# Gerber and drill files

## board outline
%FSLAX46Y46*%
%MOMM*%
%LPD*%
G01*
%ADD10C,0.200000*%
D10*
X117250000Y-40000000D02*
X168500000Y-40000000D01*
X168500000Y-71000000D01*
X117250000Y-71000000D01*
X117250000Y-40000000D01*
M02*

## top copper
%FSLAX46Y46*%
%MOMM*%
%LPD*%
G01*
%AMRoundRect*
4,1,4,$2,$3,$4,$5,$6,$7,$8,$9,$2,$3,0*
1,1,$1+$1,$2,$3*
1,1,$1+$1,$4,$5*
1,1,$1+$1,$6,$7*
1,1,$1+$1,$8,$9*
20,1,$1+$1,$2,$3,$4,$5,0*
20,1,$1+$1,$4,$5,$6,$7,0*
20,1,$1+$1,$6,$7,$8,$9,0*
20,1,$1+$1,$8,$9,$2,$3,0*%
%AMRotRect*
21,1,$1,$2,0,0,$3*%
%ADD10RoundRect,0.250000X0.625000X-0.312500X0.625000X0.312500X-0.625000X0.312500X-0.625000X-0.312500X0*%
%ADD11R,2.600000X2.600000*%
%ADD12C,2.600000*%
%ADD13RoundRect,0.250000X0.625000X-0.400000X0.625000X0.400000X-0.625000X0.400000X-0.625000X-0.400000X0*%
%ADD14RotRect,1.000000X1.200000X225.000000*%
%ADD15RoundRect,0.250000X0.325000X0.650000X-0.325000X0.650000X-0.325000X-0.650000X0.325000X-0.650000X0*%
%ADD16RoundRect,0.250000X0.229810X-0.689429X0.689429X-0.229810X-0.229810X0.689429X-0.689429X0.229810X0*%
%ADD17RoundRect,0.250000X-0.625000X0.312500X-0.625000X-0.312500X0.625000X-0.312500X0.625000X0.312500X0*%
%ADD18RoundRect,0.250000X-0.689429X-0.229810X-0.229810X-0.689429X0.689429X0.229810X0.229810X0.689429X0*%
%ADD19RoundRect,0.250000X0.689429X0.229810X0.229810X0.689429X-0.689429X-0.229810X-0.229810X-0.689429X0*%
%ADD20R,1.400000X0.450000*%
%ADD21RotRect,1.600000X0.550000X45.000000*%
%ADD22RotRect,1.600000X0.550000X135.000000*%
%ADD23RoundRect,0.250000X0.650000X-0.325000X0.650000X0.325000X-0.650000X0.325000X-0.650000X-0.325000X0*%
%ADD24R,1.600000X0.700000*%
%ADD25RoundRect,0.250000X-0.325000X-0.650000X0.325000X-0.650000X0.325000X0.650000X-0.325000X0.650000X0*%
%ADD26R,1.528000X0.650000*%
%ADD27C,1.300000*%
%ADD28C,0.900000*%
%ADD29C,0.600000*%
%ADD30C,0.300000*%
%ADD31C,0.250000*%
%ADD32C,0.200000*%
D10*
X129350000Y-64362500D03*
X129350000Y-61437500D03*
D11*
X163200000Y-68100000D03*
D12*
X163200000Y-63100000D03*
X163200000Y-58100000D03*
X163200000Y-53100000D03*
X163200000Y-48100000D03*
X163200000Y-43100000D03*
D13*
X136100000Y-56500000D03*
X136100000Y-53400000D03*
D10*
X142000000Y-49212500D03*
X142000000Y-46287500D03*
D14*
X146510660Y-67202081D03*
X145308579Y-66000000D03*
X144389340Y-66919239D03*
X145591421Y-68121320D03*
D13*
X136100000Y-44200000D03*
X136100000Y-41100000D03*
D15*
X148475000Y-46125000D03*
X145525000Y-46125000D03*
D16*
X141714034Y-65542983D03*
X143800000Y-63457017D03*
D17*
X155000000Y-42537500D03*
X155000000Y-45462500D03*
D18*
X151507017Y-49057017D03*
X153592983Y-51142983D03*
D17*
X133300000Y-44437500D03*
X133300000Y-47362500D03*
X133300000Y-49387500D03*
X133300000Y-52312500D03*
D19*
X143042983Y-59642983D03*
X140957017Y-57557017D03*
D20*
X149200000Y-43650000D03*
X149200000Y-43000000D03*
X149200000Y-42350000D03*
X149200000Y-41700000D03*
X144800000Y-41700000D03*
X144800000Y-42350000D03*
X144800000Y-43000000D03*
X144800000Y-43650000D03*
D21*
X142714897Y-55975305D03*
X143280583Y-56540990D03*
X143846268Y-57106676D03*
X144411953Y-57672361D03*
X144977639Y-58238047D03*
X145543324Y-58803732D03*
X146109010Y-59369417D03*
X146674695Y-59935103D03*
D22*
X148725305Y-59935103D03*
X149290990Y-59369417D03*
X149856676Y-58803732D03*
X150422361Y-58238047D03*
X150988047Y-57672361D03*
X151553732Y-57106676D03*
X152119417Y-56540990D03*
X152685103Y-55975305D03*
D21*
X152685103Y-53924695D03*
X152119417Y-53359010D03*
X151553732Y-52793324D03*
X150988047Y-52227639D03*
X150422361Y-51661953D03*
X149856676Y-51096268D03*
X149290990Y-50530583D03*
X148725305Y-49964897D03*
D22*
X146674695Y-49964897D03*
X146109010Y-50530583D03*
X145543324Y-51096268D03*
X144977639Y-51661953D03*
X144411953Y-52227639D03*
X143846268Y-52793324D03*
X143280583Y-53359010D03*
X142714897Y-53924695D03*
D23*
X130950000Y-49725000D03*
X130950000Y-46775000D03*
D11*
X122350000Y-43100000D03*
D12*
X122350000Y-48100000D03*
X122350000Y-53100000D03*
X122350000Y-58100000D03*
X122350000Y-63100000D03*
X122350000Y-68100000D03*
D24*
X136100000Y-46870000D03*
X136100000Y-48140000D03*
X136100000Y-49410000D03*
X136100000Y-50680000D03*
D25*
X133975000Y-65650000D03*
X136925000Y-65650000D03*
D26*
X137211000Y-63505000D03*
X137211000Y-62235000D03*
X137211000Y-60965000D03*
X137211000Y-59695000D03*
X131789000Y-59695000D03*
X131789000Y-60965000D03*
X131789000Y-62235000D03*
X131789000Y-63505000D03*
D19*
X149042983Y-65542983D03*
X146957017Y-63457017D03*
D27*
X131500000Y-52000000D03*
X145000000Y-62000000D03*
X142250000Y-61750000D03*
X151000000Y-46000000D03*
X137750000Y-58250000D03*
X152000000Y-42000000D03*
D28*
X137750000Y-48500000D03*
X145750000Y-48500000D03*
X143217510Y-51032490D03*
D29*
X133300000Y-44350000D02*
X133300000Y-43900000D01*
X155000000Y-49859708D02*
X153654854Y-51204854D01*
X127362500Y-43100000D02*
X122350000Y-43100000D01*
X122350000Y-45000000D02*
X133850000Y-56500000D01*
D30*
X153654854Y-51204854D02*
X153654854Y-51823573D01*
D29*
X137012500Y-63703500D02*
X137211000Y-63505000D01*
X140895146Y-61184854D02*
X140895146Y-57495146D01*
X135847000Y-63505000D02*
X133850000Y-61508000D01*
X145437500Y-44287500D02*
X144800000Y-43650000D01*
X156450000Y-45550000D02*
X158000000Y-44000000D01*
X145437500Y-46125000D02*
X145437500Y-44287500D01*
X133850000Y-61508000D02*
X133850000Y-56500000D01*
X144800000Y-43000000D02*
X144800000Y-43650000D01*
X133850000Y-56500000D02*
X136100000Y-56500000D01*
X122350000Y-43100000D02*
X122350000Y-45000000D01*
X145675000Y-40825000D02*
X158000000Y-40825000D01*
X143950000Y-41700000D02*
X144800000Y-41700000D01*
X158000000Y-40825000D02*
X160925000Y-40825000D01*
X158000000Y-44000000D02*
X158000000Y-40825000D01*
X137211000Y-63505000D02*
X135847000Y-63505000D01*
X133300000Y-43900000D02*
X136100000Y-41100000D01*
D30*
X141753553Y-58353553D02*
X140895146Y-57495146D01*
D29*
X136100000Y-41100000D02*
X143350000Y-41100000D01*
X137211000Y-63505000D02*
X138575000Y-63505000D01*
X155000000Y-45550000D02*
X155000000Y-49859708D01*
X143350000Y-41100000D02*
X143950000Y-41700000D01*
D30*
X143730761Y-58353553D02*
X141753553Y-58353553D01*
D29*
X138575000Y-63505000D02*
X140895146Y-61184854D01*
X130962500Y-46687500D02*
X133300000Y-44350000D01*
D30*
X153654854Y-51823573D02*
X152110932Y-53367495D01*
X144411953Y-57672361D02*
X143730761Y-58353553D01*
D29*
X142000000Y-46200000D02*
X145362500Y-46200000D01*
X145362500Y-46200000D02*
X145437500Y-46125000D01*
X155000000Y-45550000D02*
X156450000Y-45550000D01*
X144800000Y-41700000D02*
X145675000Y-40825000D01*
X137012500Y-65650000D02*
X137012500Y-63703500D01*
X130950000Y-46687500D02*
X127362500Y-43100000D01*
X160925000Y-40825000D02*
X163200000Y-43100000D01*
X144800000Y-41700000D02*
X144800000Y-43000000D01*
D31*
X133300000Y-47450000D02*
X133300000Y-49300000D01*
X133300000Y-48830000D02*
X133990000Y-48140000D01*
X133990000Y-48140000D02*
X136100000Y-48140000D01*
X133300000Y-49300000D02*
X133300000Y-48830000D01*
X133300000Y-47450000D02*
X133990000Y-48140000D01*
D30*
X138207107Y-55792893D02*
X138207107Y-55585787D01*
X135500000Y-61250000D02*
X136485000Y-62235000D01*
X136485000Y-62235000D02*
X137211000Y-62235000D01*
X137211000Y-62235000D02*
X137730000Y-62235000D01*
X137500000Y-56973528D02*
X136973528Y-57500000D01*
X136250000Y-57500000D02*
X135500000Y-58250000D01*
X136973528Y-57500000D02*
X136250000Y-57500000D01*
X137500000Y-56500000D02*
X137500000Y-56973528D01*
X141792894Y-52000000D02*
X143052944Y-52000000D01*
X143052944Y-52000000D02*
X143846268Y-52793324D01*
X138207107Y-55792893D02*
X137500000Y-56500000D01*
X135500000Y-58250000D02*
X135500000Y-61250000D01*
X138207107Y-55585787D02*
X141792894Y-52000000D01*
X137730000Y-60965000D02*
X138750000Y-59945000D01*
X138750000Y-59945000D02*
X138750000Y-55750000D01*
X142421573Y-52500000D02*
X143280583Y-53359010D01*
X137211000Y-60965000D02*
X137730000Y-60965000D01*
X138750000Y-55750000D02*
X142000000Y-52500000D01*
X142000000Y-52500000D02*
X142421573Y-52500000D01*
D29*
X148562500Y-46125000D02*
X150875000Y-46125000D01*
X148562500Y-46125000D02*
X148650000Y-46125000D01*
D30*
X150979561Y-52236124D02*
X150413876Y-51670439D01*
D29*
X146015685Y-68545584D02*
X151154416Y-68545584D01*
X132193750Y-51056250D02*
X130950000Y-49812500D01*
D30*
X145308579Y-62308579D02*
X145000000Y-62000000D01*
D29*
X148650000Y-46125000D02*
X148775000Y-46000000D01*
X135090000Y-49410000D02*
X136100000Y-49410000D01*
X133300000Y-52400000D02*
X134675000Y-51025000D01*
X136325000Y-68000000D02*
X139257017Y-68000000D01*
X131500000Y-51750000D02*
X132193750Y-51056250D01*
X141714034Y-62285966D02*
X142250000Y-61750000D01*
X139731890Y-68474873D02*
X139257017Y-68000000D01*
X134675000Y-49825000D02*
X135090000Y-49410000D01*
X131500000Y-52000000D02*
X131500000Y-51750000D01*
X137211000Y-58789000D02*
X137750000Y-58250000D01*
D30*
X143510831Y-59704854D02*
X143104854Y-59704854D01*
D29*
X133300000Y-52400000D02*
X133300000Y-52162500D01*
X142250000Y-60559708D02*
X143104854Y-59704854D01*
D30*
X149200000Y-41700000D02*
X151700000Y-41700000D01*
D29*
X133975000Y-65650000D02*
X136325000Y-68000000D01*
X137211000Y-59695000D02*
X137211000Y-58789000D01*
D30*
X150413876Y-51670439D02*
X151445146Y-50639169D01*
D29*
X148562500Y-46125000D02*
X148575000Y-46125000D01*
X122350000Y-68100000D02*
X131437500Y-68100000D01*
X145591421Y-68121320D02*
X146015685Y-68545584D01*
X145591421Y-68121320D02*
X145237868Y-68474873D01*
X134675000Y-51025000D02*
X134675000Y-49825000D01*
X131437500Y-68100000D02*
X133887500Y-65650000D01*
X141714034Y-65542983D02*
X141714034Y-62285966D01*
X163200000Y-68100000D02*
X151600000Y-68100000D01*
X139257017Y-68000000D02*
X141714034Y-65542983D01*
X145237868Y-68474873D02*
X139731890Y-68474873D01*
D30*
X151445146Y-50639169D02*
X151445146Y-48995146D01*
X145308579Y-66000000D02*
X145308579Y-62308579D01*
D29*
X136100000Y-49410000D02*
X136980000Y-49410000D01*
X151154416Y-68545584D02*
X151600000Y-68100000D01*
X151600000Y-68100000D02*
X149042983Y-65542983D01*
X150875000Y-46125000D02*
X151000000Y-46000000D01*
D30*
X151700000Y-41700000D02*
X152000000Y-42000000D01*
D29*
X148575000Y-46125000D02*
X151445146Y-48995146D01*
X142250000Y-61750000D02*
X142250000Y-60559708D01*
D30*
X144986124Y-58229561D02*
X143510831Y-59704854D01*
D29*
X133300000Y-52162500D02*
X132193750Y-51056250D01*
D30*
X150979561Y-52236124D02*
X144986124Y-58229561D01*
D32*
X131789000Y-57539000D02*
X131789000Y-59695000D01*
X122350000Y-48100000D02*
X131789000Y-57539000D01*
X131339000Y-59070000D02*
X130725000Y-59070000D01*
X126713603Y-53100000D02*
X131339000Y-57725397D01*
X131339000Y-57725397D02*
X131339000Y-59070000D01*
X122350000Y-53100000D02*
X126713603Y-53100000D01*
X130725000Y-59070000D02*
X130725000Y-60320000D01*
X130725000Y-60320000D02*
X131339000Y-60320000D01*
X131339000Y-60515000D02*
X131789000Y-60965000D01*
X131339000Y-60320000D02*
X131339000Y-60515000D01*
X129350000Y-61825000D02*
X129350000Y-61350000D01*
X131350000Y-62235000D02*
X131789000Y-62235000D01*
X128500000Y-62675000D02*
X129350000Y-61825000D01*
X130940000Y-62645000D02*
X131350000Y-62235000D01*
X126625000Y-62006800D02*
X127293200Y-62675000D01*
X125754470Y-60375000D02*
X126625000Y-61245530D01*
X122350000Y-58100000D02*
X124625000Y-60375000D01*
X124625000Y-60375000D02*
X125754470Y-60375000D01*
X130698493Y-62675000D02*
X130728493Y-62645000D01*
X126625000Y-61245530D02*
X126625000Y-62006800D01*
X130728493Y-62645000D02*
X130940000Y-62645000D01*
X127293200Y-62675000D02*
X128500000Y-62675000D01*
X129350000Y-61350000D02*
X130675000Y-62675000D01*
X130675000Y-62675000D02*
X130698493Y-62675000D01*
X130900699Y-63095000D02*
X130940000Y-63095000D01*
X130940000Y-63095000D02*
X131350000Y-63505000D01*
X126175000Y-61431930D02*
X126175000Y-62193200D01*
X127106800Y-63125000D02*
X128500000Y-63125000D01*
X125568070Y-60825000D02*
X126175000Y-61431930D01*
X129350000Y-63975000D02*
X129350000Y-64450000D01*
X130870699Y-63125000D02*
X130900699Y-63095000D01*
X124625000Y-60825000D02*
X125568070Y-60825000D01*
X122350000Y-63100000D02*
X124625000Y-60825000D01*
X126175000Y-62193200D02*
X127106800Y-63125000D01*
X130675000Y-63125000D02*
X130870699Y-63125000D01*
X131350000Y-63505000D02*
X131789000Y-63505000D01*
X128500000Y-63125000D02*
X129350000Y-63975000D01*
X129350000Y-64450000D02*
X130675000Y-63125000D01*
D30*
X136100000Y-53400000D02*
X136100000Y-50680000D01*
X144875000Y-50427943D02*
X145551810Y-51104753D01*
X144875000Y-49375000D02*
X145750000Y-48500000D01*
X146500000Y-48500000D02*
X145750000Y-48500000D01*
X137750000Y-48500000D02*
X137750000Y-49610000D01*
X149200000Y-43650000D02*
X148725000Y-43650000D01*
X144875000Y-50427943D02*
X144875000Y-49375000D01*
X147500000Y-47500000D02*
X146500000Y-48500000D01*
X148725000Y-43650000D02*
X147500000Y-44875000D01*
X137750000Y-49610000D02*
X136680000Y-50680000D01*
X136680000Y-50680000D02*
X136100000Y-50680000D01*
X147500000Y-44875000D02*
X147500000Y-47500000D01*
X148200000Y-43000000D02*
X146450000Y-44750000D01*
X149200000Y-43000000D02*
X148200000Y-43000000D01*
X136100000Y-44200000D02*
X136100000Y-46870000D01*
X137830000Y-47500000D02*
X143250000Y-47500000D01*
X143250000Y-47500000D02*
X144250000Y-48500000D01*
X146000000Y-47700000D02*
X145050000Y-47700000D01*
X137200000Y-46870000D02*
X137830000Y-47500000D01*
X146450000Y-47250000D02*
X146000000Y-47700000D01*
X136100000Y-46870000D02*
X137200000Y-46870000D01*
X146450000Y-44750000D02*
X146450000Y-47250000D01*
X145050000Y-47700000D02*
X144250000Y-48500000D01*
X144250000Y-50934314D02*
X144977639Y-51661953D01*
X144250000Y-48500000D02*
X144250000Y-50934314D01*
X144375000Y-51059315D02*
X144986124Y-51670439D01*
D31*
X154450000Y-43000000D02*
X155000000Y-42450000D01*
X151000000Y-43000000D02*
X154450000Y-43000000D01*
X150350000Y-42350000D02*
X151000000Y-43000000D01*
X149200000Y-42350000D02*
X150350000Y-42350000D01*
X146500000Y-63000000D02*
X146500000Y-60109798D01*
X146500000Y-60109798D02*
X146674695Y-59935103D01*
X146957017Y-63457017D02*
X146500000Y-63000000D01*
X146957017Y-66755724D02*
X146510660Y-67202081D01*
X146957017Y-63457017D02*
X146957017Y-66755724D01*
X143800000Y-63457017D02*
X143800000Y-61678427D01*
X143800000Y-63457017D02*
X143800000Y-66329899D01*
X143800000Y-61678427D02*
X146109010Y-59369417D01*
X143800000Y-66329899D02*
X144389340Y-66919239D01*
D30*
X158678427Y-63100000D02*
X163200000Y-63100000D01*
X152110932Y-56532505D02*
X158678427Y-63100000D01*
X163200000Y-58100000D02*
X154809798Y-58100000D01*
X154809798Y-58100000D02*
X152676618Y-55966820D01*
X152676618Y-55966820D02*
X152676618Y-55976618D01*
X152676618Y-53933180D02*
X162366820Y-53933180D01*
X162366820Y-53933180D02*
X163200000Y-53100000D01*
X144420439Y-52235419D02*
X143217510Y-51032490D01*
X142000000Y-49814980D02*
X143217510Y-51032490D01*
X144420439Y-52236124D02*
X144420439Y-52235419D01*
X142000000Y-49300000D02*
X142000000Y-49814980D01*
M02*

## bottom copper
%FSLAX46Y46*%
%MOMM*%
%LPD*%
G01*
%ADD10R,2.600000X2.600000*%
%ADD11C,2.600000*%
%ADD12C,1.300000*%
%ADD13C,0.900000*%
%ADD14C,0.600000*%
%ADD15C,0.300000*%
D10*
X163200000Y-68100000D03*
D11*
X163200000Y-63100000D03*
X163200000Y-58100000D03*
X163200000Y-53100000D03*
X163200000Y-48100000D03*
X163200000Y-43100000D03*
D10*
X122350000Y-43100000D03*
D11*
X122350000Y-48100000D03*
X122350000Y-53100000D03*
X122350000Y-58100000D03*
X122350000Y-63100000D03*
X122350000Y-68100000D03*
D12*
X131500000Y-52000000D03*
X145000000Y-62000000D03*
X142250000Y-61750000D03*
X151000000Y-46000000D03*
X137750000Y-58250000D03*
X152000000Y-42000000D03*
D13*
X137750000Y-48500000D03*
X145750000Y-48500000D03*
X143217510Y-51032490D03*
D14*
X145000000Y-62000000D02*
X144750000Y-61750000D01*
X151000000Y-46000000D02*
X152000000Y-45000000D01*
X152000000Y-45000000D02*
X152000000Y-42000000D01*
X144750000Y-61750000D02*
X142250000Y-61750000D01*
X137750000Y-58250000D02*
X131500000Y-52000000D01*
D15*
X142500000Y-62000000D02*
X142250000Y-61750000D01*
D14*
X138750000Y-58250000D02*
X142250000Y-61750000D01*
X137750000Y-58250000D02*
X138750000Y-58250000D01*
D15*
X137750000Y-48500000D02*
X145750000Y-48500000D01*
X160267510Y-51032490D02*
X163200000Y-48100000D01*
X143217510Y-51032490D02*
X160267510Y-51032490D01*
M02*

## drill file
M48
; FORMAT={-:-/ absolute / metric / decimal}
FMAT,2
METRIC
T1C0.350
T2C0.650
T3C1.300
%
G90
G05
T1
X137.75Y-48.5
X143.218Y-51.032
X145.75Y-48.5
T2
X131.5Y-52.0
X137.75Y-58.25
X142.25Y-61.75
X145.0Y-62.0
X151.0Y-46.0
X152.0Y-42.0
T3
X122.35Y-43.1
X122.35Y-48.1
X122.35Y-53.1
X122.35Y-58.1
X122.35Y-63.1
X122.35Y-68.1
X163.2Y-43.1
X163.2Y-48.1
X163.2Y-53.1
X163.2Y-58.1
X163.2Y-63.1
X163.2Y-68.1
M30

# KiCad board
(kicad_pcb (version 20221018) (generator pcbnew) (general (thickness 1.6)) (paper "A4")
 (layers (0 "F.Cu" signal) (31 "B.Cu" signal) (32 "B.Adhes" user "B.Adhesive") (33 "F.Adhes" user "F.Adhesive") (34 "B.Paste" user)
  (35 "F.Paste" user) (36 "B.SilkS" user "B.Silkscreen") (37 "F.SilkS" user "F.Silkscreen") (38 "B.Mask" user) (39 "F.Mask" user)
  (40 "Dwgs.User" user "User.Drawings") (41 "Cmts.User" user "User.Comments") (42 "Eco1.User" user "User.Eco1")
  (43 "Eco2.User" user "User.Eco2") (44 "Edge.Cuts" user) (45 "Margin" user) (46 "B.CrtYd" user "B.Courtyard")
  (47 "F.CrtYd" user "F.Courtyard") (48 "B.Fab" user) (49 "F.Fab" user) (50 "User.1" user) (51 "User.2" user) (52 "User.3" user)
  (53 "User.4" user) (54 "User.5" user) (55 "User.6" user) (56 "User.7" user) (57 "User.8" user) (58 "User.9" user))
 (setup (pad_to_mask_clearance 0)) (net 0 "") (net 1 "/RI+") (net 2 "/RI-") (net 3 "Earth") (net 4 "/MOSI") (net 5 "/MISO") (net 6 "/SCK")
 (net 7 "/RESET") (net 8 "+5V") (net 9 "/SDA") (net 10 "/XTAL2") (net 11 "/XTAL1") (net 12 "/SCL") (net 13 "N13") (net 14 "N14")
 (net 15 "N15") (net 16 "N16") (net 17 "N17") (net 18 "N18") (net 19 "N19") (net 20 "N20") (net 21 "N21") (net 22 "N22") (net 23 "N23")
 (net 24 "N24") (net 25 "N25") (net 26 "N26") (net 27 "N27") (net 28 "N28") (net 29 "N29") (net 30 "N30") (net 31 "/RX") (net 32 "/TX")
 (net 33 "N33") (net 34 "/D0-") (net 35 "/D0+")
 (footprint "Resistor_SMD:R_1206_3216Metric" (layer "F.Cu") (at 129.35 62.9 90)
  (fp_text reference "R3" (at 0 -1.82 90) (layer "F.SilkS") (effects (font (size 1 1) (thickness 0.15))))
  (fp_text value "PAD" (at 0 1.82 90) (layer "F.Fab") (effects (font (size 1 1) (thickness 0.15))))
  (pad "1" smd roundrect (at -1.4625 0 90) (size 1.125 1.75) (layers "F.Cu" "F.Paste" "F.Mask") (roundrect_rratio 0.222222) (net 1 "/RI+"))
  (pad "2" smd roundrect (at 1.4625 0 90) (size 1.125 1.75) (layers "F.Cu" "F.Paste" "F.Mask") (roundrect_rratio 0.222222) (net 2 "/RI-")))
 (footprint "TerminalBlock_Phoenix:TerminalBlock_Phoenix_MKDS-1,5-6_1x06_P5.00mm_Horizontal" (layer "F.Cu") (at 163.2 68.1 90)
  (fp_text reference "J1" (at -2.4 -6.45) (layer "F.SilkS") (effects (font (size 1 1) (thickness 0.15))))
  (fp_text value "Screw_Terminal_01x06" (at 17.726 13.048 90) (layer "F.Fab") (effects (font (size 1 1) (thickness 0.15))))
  (pad "1" thru_hole rect (at 0 0 90) (size 2.6 2.6) (drill 1.3) (layers "*.Cu" "*.Mask") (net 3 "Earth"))
  (pad "2" thru_hole circle (at 5 0 90) (size 2.6 2.6) (drill 1.3) (layers "*.Cu" "*.Mask") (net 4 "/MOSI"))
  (pad "3" thru_hole circle (at 10 0 90) (size 2.6 2.6) (drill 1.3) (layers "*.Cu" "*.Mask") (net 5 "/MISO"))
  (pad "4" thru_hole circle (at 15 0 90) (size 2.6 2.6) (drill 1.3) (layers "*.Cu" "*.Mask") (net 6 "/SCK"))
  (pad "5" thru_hole circle (at 20 0 90) (size 2.6 2.6) (drill 1.3) (layers "*.Cu" "*.Mask") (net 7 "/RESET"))
  (pad "6" thru_hole circle (at 25 0 90) (size 2.6 2.6) (drill 1.3) (layers "*.Cu" "*.Mask") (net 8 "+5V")))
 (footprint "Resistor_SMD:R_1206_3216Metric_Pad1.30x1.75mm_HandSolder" (layer "F.Cu") (at 136.1 54.95 90)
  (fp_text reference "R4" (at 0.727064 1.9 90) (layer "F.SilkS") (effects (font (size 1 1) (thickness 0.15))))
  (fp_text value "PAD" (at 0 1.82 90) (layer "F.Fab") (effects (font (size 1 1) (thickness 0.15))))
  (pad "1" smd roundrect (at -1.55 0 90) (size 1.3 1.75) (layers "F.Cu" "F.Paste" "F.Mask") (roundrect_rratio 0.192308) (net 8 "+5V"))
  (pad "2" smd roundrect (at 1.55 0 90) (size 1.3 1.75) (layers "F.Cu" "F.Paste" "F.Mask") (roundrect_rratio 0.192308) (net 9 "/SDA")))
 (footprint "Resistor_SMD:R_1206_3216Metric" (layer "F.Cu") (at 142 47.75 90)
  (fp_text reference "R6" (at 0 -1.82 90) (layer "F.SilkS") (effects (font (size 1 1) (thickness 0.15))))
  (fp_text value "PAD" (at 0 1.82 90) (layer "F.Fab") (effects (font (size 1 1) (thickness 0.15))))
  (pad "1" smd roundrect (at -1.4625 0 90) (size 1.125 1.75) (layers "F.Cu" "F.Paste" "F.Mask") (roundrect_rratio 0.222222) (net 7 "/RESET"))
  (pad "2" smd roundrect (at 1.4625 0 90) (size 1.125 1.75) (layers "F.Cu" "F.Paste" "F.Mask") (roundrect_rratio 0.222222) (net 8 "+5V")))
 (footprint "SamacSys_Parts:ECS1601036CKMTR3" (layer "F.Cu") (at 145.45 67.06066 135)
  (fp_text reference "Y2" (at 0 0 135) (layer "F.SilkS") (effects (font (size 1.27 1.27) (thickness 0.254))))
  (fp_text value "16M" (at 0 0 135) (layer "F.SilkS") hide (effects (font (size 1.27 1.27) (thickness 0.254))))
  (pad "1" smd rect (at -0.85 0.65 225) (size 1 1.2) (layers "F.Cu" "F.Paste" "F.Mask") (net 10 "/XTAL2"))
  (pad "2" smd rect (at 0.85 0.65 225) (size 1 1.2) (layers "F.Cu" "F.Paste" "F.Mask") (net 3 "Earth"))
  (pad "3" smd rect (at 0.85 -0.65 225) (size 1 1.2) (layers "F.Cu" "F.Paste" "F.Mask") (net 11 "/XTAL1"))
  (pad "4" smd rect (at -0.85 -0.65 225) (size 1 1.2) (layers "F.Cu" "F.Paste" "F.Mask") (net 3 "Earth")))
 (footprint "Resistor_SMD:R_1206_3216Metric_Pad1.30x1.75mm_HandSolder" (layer "F.Cu") (at 136.1 42.65 90)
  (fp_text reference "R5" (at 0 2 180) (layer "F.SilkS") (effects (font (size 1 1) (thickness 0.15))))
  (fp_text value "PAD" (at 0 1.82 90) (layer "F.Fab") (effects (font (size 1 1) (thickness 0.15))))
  (pad "1" smd roundrect (at -1.55 0 90) (size 1.3 1.75) (layers "F.Cu" "F.Paste" "F.Mask") (roundrect_rratio 0.192308) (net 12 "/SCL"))
  (pad "2" smd roundrect (at 1.55 0 90) (size 1.3 1.75) (layers "F.Cu" "F.Paste" "F.Mask") (roundrect_rratio 0.192308) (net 8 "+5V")))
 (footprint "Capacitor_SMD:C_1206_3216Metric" (layer "F.Cu") (at 147 46.125 180)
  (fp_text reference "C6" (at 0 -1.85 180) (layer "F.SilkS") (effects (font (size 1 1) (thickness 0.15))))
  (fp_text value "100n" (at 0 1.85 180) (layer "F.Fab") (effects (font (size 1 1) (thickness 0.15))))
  (pad "1" smd roundrect (at -1.475 0 180) (size 1.15 1.8) (layers "F.Cu" "F.Paste" "F.Mask") (roundrect_rratio 0.217391) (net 3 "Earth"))
  (pad "2" smd roundrect (at 1.475 0 180) (size 1.15 1.8) (layers "F.Cu" "F.Paste" "F.Mask") (roundrect_rratio 0.217391) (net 8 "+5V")))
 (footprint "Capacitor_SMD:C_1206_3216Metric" (layer "F.Cu") (at 142.757017 64.5 45)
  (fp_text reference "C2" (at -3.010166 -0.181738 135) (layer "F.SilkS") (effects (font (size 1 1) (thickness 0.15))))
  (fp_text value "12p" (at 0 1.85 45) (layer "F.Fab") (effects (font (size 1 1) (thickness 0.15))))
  (pad "1" smd roundrect (at -1.475 0 45) (size 1.15 1.8) (layers "F.Cu" "F.Paste" "F.Mask") (roundrect_rratio 0.217391) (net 3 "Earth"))
  (pad "2" smd roundrect (at 1.475 0 45) (size 1.15 1.8) (layers "F.Cu" "F.Paste" "F.Mask") (roundrect_rratio 0.217391) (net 11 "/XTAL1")))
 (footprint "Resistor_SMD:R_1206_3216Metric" (layer "F.Cu") (at 155 44 -90)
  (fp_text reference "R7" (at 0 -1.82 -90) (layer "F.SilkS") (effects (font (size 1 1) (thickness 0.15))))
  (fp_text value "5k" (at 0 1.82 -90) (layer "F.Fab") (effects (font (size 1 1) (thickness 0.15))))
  (pad "1" smd roundrect (at -1.4625 0 270) (size 1.125 1.75) (layers "F.Cu" "F.Paste" "F.Mask") (roundrect_rratio 0.222222) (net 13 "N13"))
  (pad "2" smd roundrect (at 1.4625 0 270) (size 1.125 1.75) (layers "F.Cu" "F.Paste" "F.Mask") (roundrect_rratio 0.222222) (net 8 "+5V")))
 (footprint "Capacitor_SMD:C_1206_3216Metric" (layer "F.Cu") (at 152.55 50.1 -45)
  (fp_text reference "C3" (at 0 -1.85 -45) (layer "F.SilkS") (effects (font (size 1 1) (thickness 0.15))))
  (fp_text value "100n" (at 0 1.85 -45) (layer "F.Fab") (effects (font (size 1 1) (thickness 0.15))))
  (pad "1" smd roundrect (at -1.475 0 315) (size 1.15 1.8) (layers "F.Cu" "F.Paste" "F.Mask") (roundrect_rratio 0.217391) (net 3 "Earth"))
  (pad "2" smd roundrect (at 1.475 0 315) (size 1.15 1.8) (layers "F.Cu" "F.Paste" "F.Mask") (roundrect_rratio 0.217391) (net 8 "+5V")))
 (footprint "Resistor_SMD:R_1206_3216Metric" (layer "F.Cu") (at 133.3 45.9 -90)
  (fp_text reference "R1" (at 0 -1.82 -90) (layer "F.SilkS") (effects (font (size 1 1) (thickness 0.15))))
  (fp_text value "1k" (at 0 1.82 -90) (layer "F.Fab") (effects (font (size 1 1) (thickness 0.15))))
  (pad "1" smd roundrect (at -1.4625 0 270) (size 1.125 1.75) (layers "F.Cu" "F.Paste" "F.Mask") (roundrect_rratio 0.222222) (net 8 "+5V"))
  (pad "2" smd roundrect (at 1.4625 0 270) (size 1.125 1.75) (layers "F.Cu" "F.Paste" "F.Mask") (roundrect_rratio 0.222222) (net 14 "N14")))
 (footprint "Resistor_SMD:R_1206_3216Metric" (layer "F.Cu") (at 133.3 50.85 -90)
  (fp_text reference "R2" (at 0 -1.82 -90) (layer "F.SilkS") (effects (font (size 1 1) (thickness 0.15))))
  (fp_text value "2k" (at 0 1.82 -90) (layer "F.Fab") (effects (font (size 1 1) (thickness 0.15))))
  (pad "1" smd roundrect (at -1.4625 0 270) (size 1.125 1.75) (layers "F.Cu" "F.Paste" "F.Mask") (roundrect_rratio 0.222222) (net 14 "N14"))
  (pad "2" smd roundrect (at 1.4625 0 270) (size 1.125 1.75) (layers "F.Cu" "F.Paste" "F.Mask") (roundrect_rratio 0.222222) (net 3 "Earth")))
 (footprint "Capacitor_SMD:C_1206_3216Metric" (layer "F.Cu") (at 142 58.6 135)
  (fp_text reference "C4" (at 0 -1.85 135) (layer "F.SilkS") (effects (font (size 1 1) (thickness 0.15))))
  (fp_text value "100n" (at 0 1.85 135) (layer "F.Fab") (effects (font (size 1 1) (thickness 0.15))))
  (pad "1" smd roundrect (at -1.475 0 135) (size 1.15 1.8) (layers "F.Cu" "F.Paste" "F.Mask") (roundrect_rratio 0.217391) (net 3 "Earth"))
  (pad "2" smd roundrect (at 1.475 0 135) (size 1.15 1.8) (layers "F.Cu" "F.Paste" "F.Mask") (roundrect_rratio 0.217391) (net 8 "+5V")))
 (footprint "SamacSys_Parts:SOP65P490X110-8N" (layer "F.Cu") (at 147 42.675 180)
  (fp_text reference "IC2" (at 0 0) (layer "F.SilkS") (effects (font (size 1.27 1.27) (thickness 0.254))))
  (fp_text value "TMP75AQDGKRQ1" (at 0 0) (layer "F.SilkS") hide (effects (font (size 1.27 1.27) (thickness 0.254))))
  (pad "1" smd rect (at -2.2 -0.975 270) (size 0.45 1.4) (layers "F.Cu" "F.Paste" "F.Mask") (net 9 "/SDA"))
  (pad "2" smd rect (at -2.2 -0.325 270) (size 0.45 1.4) (layers "F.Cu" "F.Paste" "F.Mask") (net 12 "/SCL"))
  (pad "3" smd rect (at -2.2 0.325 270) (size 0.45 1.4) (layers "F.Cu" "F.Paste" "F.Mask") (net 13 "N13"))
  (pad "4" smd rect (at -2.2 0.975 270) (size 0.45 1.4) (layers "F.Cu" "F.Paste" "F.Mask") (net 3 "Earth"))
  (pad "5" smd rect (at 2.2 0.975 270) (size 0.45 1.4) (layers "F.Cu" "F.Paste" "F.Mask") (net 8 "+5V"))
  (pad "6" smd rect (at 2.2 0.325 270) (size 0.45 1.4) (layers "F.Cu" "F.Paste" "F.Mask") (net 8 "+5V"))
  (pad "7" smd rect (at 2.2 -0.325 270) (size 0.45 1.4) (layers "F.Cu" "F.Paste" "F.Mask") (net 8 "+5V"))
  (pad "8" smd rect (at 2.2 -0.975 270) (size 0.45 1.4) (layers "F.Cu" "F.Paste" "F.Mask") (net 8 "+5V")))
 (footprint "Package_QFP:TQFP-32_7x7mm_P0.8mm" (layer "F.Cu") (at 147.7 54.95 45)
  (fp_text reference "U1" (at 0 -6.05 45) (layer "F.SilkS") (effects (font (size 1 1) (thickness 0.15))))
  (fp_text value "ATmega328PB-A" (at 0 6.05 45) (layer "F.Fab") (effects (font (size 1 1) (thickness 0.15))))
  (pad "1" smd rect (at -4.25 -2.8 45) (size 1.6 0.55) (layers "F.Cu" "F.Paste" "F.Mask") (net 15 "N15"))
  (pad "2" smd rect (at -4.25 -2 45) (size 1.6 0.55) (layers "F.Cu" "F.Paste" "F.Mask") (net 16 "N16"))
  (pad "3" smd rect (at -4.25 -1.2 45) (size 1.6 0.55) (layers "F.Cu" "F.Paste" "F.Mask") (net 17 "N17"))
  (pad "4" smd rect (at -4.25 -0.4 45) (size 1.6 0.55) (layers "F.Cu" "F.Paste" "F.Mask") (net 8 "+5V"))
  (pad "5" smd rect (at -4.25 0.4 45) (size 1.6 0.55) (layers "F.Cu" "F.Paste" "F.Mask") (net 3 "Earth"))
  (pad "6" smd rect (at -4.25 1.2 45) (size 1.6 0.55) (layers "F.Cu" "F.Paste" "F.Mask") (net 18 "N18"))
  (pad "7" smd rect (at -4.25 2 45) (size 1.6 0.55) (layers "F.Cu" "F.Paste" "F.Mask") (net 11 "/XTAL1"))
  (pad "8" smd rect (at -4.25 2.8 45) (size 1.6 0.55) (layers "F.Cu" "F.Paste" "F.Mask") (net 10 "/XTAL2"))
  (pad "9" smd rect (at -2.8 4.25 135) (size 1.6 0.55) (layers "F.Cu" "F.Paste" "F.Mask") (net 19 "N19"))
  (pad "10" smd rect (at -2 4.25 135) (size 1.6 0.55) (layers "F.Cu" "F.Paste" "F.Mask") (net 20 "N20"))
  (pad "11" smd rect (at -1.2 4.25 135) (size 1.6 0.55) (layers "F.Cu" "F.Paste" "F.Mask") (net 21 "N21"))
  (pad "12" smd rect (at -0.4 4.25 135) (size 1.6 0.55) (layers "F.Cu" "F.Paste" "F.Mask") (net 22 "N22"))
  (pad "13" smd rect (at 0.4 4.25 135) (size 1.6 0.55) (layers "F.Cu" "F.Paste" "F.Mask") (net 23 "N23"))
  (pad "14" smd rect (at 1.2 4.25 135) (size 1.6 0.55) (layers "F.Cu" "F.Paste" "F.Mask") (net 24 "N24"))
  (pad "15" smd rect (at 2 4.25 135) (size 1.6 0.55) (layers "F.Cu" "F.Paste" "F.Mask") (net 4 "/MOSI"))
  (pad "16" smd rect (at 2.8 4.25 135) (size 1.6 0.55) (layers "F.Cu" "F.Paste" "F.Mask") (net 5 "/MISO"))
  (pad "17" smd rect (at 4.25 2.8 45) (size 1.6 0.55) (layers "F.Cu" "F.Paste" "F.Mask") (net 6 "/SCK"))
  (pad "18" smd rect (at 4.25 2 45) (size 1.6 0.55) (layers "F.Cu" "F.Paste" "F.Mask") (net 8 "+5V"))
  (pad "19" smd rect (at 4.25 1.2 45) (size 1.6 0.55) (layers "F.Cu" "F.Paste" "F.Mask") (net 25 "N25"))
  (pad "20" smd rect (at 4.25 0.4 45) (size 1.6 0.55) (layers "F.Cu" "F.Paste" "F.Mask") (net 3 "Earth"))
  (pad "21" smd rect (at 4.25 -0.4 45) (size 1.6 0.55) (layers "F.Cu" "F.Paste" "F.Mask") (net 3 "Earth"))
  (pad "22" smd rect (at 4.25 -1.2 45) (size 1.6 0.55) (layers "F.Cu" "F.Paste" "F.Mask") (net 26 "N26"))
  (pad "23" smd rect (at 4.25 -2 45) (size 1.6 0.55) (layers "F.Cu" "F.Paste" "F.Mask") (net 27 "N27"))
  (pad "24" smd rect (at 4.25 -2.8 45) (size 1.6 0.55) (layers "F.Cu" "F.Paste" "F.Mask") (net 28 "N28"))
  (pad "25" smd rect (at 2.8 -4.25 135) (size 1.6 0.55) (layers "F.Cu" "F.Paste" "F.Mask") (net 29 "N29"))
  (pad "26" smd rect (at 2 -4.25 135) (size 1.6 0.55) (layers "F.Cu" "F.Paste" "F.Mask") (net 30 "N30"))
  (pad "27" smd rect (at 1.2 -4.25 135) (size 1.6 0.55) (layers "F.Cu" "F.Paste" "F.Mask") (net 9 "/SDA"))
  (pad "28" smd rect (at 0.4 -4.25 135) (size 1.6 0.55) (layers "F.Cu" "F.Paste" "F.Mask") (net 12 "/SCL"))
  (pad "29" smd rect (at -0.4 -4.25 135) (size 1.6 0.55) (layers "F.Cu" "F.Paste" "F.Mask") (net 7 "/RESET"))
  (pad "30" smd rect (at -1.2 -4.25 135) (size 1.6 0.55) (layers "F.Cu" "F.Paste" "F.Mask") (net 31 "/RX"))
  (pad "31" smd rect (at -2 -4.25 135) (size 1.6 0.55) (layers "F.Cu" "F.Paste" "F.Mask") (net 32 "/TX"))
  (pad "32" smd rect (at -2.8 -4.25 135) (size 1.6 0.55) (layers "F.Cu" "F.Paste" "F.Mask") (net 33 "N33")))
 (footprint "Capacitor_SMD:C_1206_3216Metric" (layer "F.Cu") (at 130.95 48.25 90)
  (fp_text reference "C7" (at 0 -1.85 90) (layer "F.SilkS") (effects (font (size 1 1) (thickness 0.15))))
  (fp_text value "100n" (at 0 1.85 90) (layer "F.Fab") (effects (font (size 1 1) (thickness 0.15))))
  (pad "1" smd roundrect (at -1.475 0 90) (size 1.15 1.8) (layers "F.Cu" "F.Paste" "F.Mask") (roundrect_rratio 0.217391) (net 3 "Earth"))
  (pad "2" smd roundrect (at 1.475 0 90) (size 1.15 1.8) (layers "F.Cu" "F.Paste" "F.Mask") (roundrect_rratio 0.217391) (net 8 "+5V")))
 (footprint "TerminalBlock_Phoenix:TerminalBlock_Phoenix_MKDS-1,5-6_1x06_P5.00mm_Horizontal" (layer "F.Cu") (at 122.35 43.1 -90)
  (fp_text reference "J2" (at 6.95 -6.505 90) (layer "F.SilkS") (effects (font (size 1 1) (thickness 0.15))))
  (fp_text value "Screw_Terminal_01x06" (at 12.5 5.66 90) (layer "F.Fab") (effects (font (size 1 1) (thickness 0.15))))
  (pad "1" thru_hole rect (at 0 0 270) (size 2.6 2.6) (drill 1.3) (layers "*.Cu" "*.Mask") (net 8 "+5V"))
  (pad "2" thru_hole circle (at 5 0 270) (size 2.6 2.6) (drill 1.3) (layers "*.Cu" "*.Mask") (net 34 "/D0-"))
  (pad "3" thru_hole circle (at 10 0 270) (size 2.6 2.6) (drill 1.3) (layers "*.Cu" "*.Mask") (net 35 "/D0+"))
  (pad "4" thru_hole circle (at 15 0 270) (size 2.6 2.6) (drill 1.3) (layers "*.Cu" "*.Mask") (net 2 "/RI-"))
  (pad "5" thru_hole circle (at 20 0 270) (size 2.6 2.6) (drill 1.3) (layers "*.Cu" "*.Mask") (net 1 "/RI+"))
  (pad "6" thru_hole circle (at 25 0 270) (size 2.6 2.6) (drill 1.3) (layers "*.Cu" "*.Mask") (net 3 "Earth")))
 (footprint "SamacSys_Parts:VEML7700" (layer "F.Cu") (at 136.5 45.375 -90)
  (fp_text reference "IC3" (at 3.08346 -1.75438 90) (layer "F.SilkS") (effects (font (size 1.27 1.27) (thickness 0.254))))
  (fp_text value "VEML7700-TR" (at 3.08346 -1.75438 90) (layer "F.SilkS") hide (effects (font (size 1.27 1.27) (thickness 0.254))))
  (pad "1" smd rect (at 1.495 0.4 270) (size 0.7 1.6) (layers "F.Cu" "F.Paste" "F.Mask") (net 12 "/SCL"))
  (pad "2" smd rect (at 2.765 0.4 270) (size 0.7 1.6) (layers "F.Cu" "F.Paste" "F.Mask") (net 14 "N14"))
  (pad "3" smd rect (at 4.035 0.4 270) (size 0.7 1.6) (layers "F.Cu" "F.Paste" "F.Mask") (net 3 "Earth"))
  (pad "4" smd rect (at 5.305 0.4 270) (size 0.7 1.6) (layers "F.Cu" "F.Paste" "F.Mask") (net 9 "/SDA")))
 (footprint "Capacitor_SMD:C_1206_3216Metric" (layer "F.Cu") (at 135.45 65.65)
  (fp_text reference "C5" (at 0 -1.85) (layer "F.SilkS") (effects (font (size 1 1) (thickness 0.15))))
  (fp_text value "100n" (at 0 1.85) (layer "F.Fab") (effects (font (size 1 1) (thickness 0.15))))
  (pad "1" smd roundrect (at -1.475 0) (size 1.15 1.8) (layers "F.Cu" "F.Paste" "F.Mask") (roundrect_rratio 0.217391) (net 3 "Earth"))
  (pad "2" smd roundrect (at 1.475 0) (size 1.15 1.8) (layers "F.Cu" "F.Paste" "F.Mask") (roundrect_rratio 0.217391) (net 8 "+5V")))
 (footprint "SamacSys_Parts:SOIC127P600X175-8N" (layer "F.Cu") (at 134.5 61.6 180)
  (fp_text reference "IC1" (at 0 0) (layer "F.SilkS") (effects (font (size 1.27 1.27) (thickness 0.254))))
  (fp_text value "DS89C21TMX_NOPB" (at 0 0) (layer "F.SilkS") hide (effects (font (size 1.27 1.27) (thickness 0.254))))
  (pad "1" smd rect (at -2.711 -1.905 270) (size 0.65 1.528) (layers "F.Cu" "F.Paste" "F.Mask") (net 8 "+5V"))
  (pad "2" smd rect (at -2.711 -0.635 270) (size 0.65 1.528) (layers "F.Cu" "F.Paste" "F.Mask") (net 31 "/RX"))
  (pad "3" smd rect (at -2.711 0.635 270) (size 0.65 1.528) (layers "F.Cu" "F.Paste" "F.Mask") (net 32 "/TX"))
  (pad "4" smd rect (at -2.711 1.905 270) (size 0.65 1.528) (layers "F.Cu" "F.Paste" "F.Mask") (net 3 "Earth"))
  (pad "5" smd rect (at 2.711 1.905 270) (size 0.65 1.528) (layers "F.Cu" "F.Paste" "F.Mask") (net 34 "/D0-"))
  (pad "6" smd rect (at 2.711 0.635 270) (size 0.65 1.528) (layers "F.Cu" "F.Paste" "F.Mask") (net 35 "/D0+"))
  (pad "7" smd rect (at 2.711 -0.635 270) (size 0.65 1.528) (layers "F.Cu" "F.Paste" "F.Mask") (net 2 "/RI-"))
  (pad "8" smd rect (at 2.711 -1.905 270) (size 0.65 1.528) (layers "F.Cu" "F.Paste" "F.Mask") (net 1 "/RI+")))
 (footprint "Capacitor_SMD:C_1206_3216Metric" (layer "F.Cu") (at 148 64.5 135)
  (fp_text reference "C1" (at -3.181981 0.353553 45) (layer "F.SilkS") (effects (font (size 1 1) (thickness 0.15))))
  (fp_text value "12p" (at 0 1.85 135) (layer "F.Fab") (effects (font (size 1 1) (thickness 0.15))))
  (pad "1" smd roundrect (at -1.475 0 135) (size 1.15 1.8) (layers "F.Cu" "F.Paste" "F.Mask") (roundrect_rratio 0.217391) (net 3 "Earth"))
  (pad "2" smd roundrect (at 1.475 0 135) (size 1.15 1.8) (layers "F.Cu" "F.Paste" "F.Mask") (roundrect_rratio 0.217391) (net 10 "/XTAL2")))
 (gr_rect (start 117.25 40) (end 168.5 71) (stroke (width 0.2) (type default)) (fill none) (layer "Edge.Cuts"))
 (segment (start 133.3 44.35) (end 133.3 43.9) (width 0.6) (layer "F.Cu") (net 8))
 (segment (start 155 49.859708) (end 153.654854 51.204854) (width 0.6) (layer "F.Cu") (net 8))
 (segment (start 127.3625 43.1) (end 122.35 43.1) (width 0.6) (layer "F.Cu") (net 8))
 (segment (start 122.35 45) (end 133.85 56.5) (width 0.6) (layer "F.Cu") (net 8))
 (segment (start 153.654854 51.204854) (end 153.654854 51.823573) (width 0.3) (layer "F.Cu") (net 8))
 (segment (start 137.0125 63.7035) (end 137.211 63.505) (width 0.6) (layer "F.Cu") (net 8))
 (segment (start 140.895146 61.184854) (end 140.895146 57.495146) (width 0.6) (layer "F.Cu") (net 8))
 (segment (start 135.847 63.505) (end 133.85 61.508) (width 0.6) (layer "F.Cu") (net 8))
 (segment (start 145.4375 44.2875) (end 144.8 43.65) (width 0.6) (layer "F.Cu") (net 8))
 (segment (start 156.45 45.55) (end 158 44) (width 0.6) (layer "F.Cu") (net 8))
 (segment (start 145.4375 46.125) (end 145.4375 44.2875) (width 0.6) (layer "F.Cu") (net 8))
 (segment (start 133.85 61.508) (end 133.85 56.5) (width 0.6) (layer "F.Cu") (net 8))
 (segment (start 144.8 43) (end 144.8 43.65) (width 0.6) (layer "F.Cu") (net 8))
 (segment (start 133.85 56.5) (end 136.1 56.5) (width 0.6) (layer "F.Cu") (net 8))
 (segment (start 122.35 43.1) (end 122.35 45) (width 0.6) (layer "F.Cu") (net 8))
 (segment (start 145.675 40.825) (end 158 40.825) (width 0.6) (layer "F.Cu") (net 8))
 (segment (start 143.95 41.7) (end 144.8 41.7) (width 0.6) (layer "F.Cu") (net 8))
 (segment (start 158 40.825) (end 160.925 40.825) (width 0.6) (layer "F.Cu") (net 8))
 (segment (start 158 44) (end 158 40.825) (width 0.6) (layer "F.Cu") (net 8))
 (segment (start 137.211 63.505) (end 135.847 63.505) (width 0.6) (layer "F.Cu") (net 8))
 (segment (start 133.3 43.9) (end 136.1 41.1) (width 0.6) (layer "F.Cu") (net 8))
 (segment (start 141.753553 58.353553) (end 140.895146 57.495146) (width 0.3) (layer "F.Cu") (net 8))
 (segment (start 136.1 41.1) (end 143.35 41.1) (width 0.6) (layer "F.Cu") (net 8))
 (segment (start 137.211 63.505) (end 138.575 63.505) (width 0.6) (layer "F.Cu") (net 8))
 (segment (start 155 45.55) (end 155 49.859708) (width 0.6) (layer "F.Cu") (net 8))
 (segment (start 143.35 41.1) (end 143.95 41.7) (width 0.6) (layer "F.Cu") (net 8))
 (segment (start 143.730761 58.353553) (end 141.753553 58.353553) (width 0.3) (layer "F.Cu") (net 8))
 (segment (start 138.575 63.505) (end 140.895146 61.184854) (width 0.6) (layer "F.Cu") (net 8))
 (segment (start 130.9625 46.6875) (end 133.3 44.35) (width 0.6) (layer "F.Cu") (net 8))
 (segment (start 153.654854 51.823573) (end 152.110932 53.367495) (width 0.3) (layer "F.Cu") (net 8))
 (segment (start 144.411953 57.672361) (end 143.730761 58.353553) (width 0.3) (layer "F.Cu") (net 8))
 (segment (start 142 46.2) (end 145.3625 46.2) (width 0.6) (layer "F.Cu") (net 8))
 (segment (start 145.3625 46.2) (end 145.4375 46.125) (width 0.6) (layer "F.Cu") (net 8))
 (segment (start 155 45.55) (end 156.45 45.55) (width 0.6) (layer "F.Cu") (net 8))
 (segment (start 144.8 41.7) (end 145.675 40.825) (width 0.6) (layer "F.Cu") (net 8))
 (segment (start 137.0125 65.65) (end 137.0125 63.7035) (width 0.6) (layer "F.Cu") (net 8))
 (segment (start 130.95 46.6875) (end 127.3625 43.1) (width 0.6) (layer "F.Cu") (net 8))
 (segment (start 160.925 40.825) (end 163.2 43.1) (width 0.6) (layer "F.Cu") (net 8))
 (segment (start 144.8 41.7) (end 144.8 43) (width 0.6) (layer "F.Cu") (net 8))
 (segment (start 133.3 47.45) (end 133.3 49.3) (width 0.25) (layer "F.Cu") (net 14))
 (segment (start 133.3 48.83) (end 133.99 48.14) (width 0.25) (layer "F.Cu") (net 14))
 (segment (start 133.99 48.14) (end 136.1 48.14) (width 0.25) (layer "F.Cu") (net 14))
 (segment (start 133.3 49.3) (end 133.3 48.83) (width 0.25) (layer "F.Cu") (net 14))
 (segment (start 133.3 47.45) (end 133.99 48.14) (width 0.25) (layer "F.Cu") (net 14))
 (segment (start 138.207107 55.792893) (end 138.207107 55.585787) (width 0.3) (layer "F.Cu") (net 31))
 (segment (start 135.5 61.25) (end 136.485 62.235) (width 0.3) (layer "F.Cu") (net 31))
 (segment (start 136.485 62.235) (end 137.211 62.235) (width 0.3) (layer "F.Cu") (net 31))
 (segment (start 137.211 62.235) (end 137.73 62.235) (width 0.3) (layer "F.Cu") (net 31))
 (segment (start 137.5 56.973528) (end 136.973528 57.5) (width 0.3) (layer "F.Cu") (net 31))
 (segment (start 136.25 57.5) (end 135.5 58.25) (width 0.3) (layer "F.Cu") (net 31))
 (segment (start 136.973528 57.5) (end 136.25 57.5) (width 0.3) (layer "F.Cu") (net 31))
 (segment (start 137.5 56.5) (end 137.5 56.973528) (width 0.3) (layer "F.Cu") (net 31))
 (segment (start 141.792894 52) (end 143.052944 52) (width 0.3) (layer "F.Cu") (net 31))
 (segment (start 143.052944 52) (end 143.846268 52.793324) (width 0.3) (layer "F.Cu") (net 31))
 (segment (start 138.207107 55.792893) (end 137.5 56.5) (width 0.3) (layer "F.Cu") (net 31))
 (segment (start 135.5 58.25) (end 135.5 61.25) (width 0.3) (layer "F.Cu") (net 31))
 (segment (start 138.207107 55.585787) (end 141.792894 52) (width 0.3) (layer "F.Cu") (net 31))
 (segment (start 137.73 60.965) (end 138.75 59.945) (width 0.3) (layer "F.Cu") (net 32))
 (segment (start 138.75 59.945) (end 138.75 55.75) (width 0.3) (layer "F.Cu") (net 32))
 (segment (start 142.421573 52.5) (end 143.280583 53.35901) (width 0.3) (layer "F.Cu") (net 32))
 (segment (start 137.211 60.965) (end 137.73 60.965) (width 0.3) (layer "F.Cu") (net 32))
 (segment (start 138.75 55.75) (end 142 52.5) (width 0.3) (layer "F.Cu") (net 32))
 (segment (start 142 52.5) (end 142.421573 52.5) (width 0.3) (layer "F.Cu") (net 32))
 (segment (start 148.5625 46.125) (end 150.875 46.125) (width 0.6) (layer "F.Cu") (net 3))
 (segment (start 148.5625 46.125) (end 148.65 46.125) (width 0.6) (layer "F.Cu") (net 3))
 (segment (start 150.979561 52.236124) (end 150.413876 51.670439) (width 0.3) (layer "F.Cu") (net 3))
 (segment (start 146.015685 68.545584) (end 151.154416 68.545584) (width 0.6) (layer "F.Cu") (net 3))
 (segment (start 132.19375 51.05625) (end 130.95 49.8125) (width 0.6) (layer "F.Cu") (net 3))
 (segment (start 145.308579 62.308579) (end 145 62) (width 0.3) (layer "F.Cu") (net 3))
 (segment (start 148.65 46.125) (end 148.775 46) (width 0.6) (layer "F.Cu") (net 3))
 (segment (start 135.09 49.41) (end 136.1 49.41) (width 0.6) (layer "F.Cu") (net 3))
 (segment (start 133.3 52.4) (end 134.675 51.025) (width 0.6) (layer "F.Cu") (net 3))
 (segment (start 136.325 68) (end 139.257017 68) (width 0.6) (layer "F.Cu") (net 3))
 (segment (start 131.5 51.75) (end 132.19375 51.05625) (width 0.6) (layer "F.Cu") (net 3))
 (segment (start 141.714034 62.285966) (end 142.25 61.75) (width 0.6) (layer "F.Cu") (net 3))
 (segment (start 139.73189 68.474873) (end 139.257017 68) (width 0.6) (layer "F.Cu") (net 3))
 (segment (start 134.675 49.825) (end 135.09 49.41) (width 0.6) (layer "F.Cu") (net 3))
 (segment (start 131.5 52) (end 131.5 51.75) (width 0.6) (layer "F.Cu") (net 3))
 (segment (start 137.211 58.789) (end 137.75 58.25) (width 0.6) (layer "F.Cu") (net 3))
 (segment (start 143.510831 59.704854) (end 143.104854 59.704854) (width 0.3) (layer "F.Cu") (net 3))
 (segment (start 133.3 52.4) (end 133.3 52.1625) (width 0.6) (layer "F.Cu") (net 3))
 (segment (start 142.25 60.559708) (end 143.104854 59.704854) (width 0.6) (layer "F.Cu") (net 3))
 (segment (start 149.2 41.7) (end 151.7 41.7) (width 0.3) (layer "F.Cu") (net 3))
 (segment (start 133.975 65.65) (end 136.325 68) (width 0.6) (layer "F.Cu") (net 3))
 (segment (start 137.211 59.695) (end 137.211 58.789) (width 0.6) (layer "F.Cu") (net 3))
 (segment (start 150.413876 51.670439) (end 151.445146 50.639169) (width 0.3) (layer "F.Cu") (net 3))
 (segment (start 148.5625 46.125) (end 148.575 46.125) (width 0.6) (layer "F.Cu") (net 3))
 (segment (start 122.35 68.1) (end 131.4375 68.1) (width 0.6) (layer "F.Cu") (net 3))
 (segment (start 145.591421 68.12132) (end 146.015685 68.545584) (width 0.6) (layer "F.Cu") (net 3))
 (segment (start 145.591421 68.12132) (end 145.237868 68.474873) (width 0.6) (layer "F.Cu") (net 3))
 (segment (start 134.675 51.025) (end 134.675 49.825) (width 0.6) (layer "F.Cu") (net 3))
 (segment (start 131.4375 68.1) (end 133.8875 65.65) (width 0.6) (layer "F.Cu") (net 3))
 (segment (start 141.714034 65.542983) (end 141.714034 62.285966) (width 0.6) (layer "F.Cu") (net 3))
 (segment (start 163.2 68.1) (end 151.6 68.1) (width 0.6) (layer "F.Cu") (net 3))
 (segment (start 139.257017 68) (end 141.714034 65.542983) (width 0.6) (layer "F.Cu") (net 3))
 (segment (start 145.237868 68.474873) (end 139.73189 68.474873) (width 0.6) (layer "F.Cu") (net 3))
 (segment (start 151.445146 50.639169) (end 151.445146 48.995146) (width 0.3) (layer "F.Cu") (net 3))
 (segment (start 145.308579 66) (end 145.308579 62.308579) (width 0.3) (layer "F.Cu") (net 3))
 (segment (start 136.1 49.41) (end 136.98 49.41) (width 0.6) (layer "F.Cu") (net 3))
 (segment (start 151.154416 68.545584) (end 151.6 68.1) (width 0.6) (layer "F.Cu") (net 3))
 (segment (start 151.6 68.1) (end 149.042983 65.542983) (width 0.6) (layer "F.Cu") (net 3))
 (segment (start 150.875 46.125) (end 151 46) (width 0.6) (layer "F.Cu") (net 3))
 (segment (start 151.7 41.7) (end 152 42) (width 0.3) (layer "F.Cu") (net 3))
 (segment (start 148.575 46.125) (end 151.445146 48.995146) (width 0.6) (layer "F.Cu") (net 3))
 (segment (start 142.25 61.75) (end 142.25 60.559708) (width 0.6) (layer "F.Cu") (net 3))
 (segment (start 144.986124 58.229561) (end 143.510831 59.704854) (width 0.3) (layer "F.Cu") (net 3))
 (segment (start 133.3 52.1625) (end 132.19375 51.05625) (width 0.6) (layer "F.Cu") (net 3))
 (segment (start 150.979561 52.236124) (end 144.986124 58.229561) (width 0.3) (layer "F.Cu") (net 3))
 (via (at 131.5 52) (size 1.3) (drill 0.65) (layers "F.Cu" "B.Cu") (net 3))
 (via (at 145 62) (size 1.3) (drill 0.65) (layers "F.Cu" "B.Cu") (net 3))
 (via (at 142.25 61.75) (size 1.3) (drill 0.65) (layers "F.Cu" "B.Cu") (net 3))
 (via (at 151 46) (size 1.3) (drill 0.65) (layers "F.Cu" "B.Cu") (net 3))
 (via (at 137.75 58.25) (size 1.3) (drill 0.65) (layers "F.Cu" "B.Cu") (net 3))
 (via (at 152 42) (size 1.3) (drill 0.65) (layers "F.Cu" "B.Cu") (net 3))
 (segment (start 145 62) (end 144.75 61.75) (width 0.6) (layer "B.Cu") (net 3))
 (segment (start 151 46) (end 152 45) (width 0.6) (layer "B.Cu") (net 3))
 (segment (start 152 45) (end 152 42) (width 0.6) (layer "B.Cu") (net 3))
 (segment (start 144.75 61.75) (end 142.25 61.75) (width 0.6) (layer "B.Cu") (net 3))
 (segment (start 137.75 58.25) (end 131.5 52) (width 0.6) (layer "B.Cu") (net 3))
 (segment (start 142.5 62) (end 142.25 61.75) (width 0.3) (layer "B.Cu") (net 3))
 (segment (start 138.75 58.25) (end 142.25 61.75) (width 0.6) (layer "B.Cu") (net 3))
 (segment (start 137.75 58.25) (end 138.75 58.25) (width 0.6) (layer "B.Cu") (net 3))
 (segment (start 131.789 57.539) (end 131.789 59.695) (width 0.2) (layer "F.Cu") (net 34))
 (segment (start 122.35 48.1) (end 131.789 57.539) (width 0.2) (layer "F.Cu") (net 34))
 (segment (start 131.339 59.07) (end 130.725 59.07) (width 0.2) (layer "F.Cu") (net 35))
 (segment (start 126.713603 53.1) (end 131.339 57.725397) (width 0.2) (layer "F.Cu") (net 35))
 (segment (start 131.339 57.725397) (end 131.339 59.07) (width 0.2) (layer "F.Cu") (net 35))
 (segment (start 122.35 53.1) (end 126.713603 53.1) (width 0.2) (layer "F.Cu") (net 35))
 (segment (start 130.725 59.07) (end 130.725 60.32) (width 0.2) (layer "F.Cu") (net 35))
 (segment (start 130.725 60.32) (end 131.339 60.32) (width 0.2) (layer "F.Cu") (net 35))
 (segment (start 131.339 60.515) (end 131.789 60.965) (width 0.2) (layer "F.Cu") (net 35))
 (segment (start 131.339 60.32) (end 131.339 60.515) (width 0.2) (layer "F.Cu") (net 35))
 (segment (start 129.35 61.825) (end 129.35 61.35) (width 0.2) (layer "F.Cu") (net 2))
 (segment (start 131.35 62.235) (end 131.789 62.235) (width 0.2) (layer "F.Cu") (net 2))
 (segment (start 128.5 62.675) (end 129.35 61.825) (width 0.2) (layer "F.Cu") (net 2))
 (segment (start 130.94 62.645) (end 131.35 62.235) (width 0.2) (layer "F.Cu") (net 2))
 (segment (start 126.625 62.0068) (end 127.2932 62.675) (width 0.2) (layer "F.Cu") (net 2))
 (segment (start 125.75447 60.375) (end 126.625 61.24553) (width 0.2) (layer "F.Cu") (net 2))
 (segment (start 122.35 58.1) (end 124.625 60.375) (width 0.2) (layer "F.Cu") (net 2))
 (segment (start 124.625 60.375) (end 125.75447 60.375) (width 0.2) (layer "F.Cu") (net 2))
 (segment (start 130.698493 62.675) (end 130.728493 62.645) (width 0.2) (layer "F.Cu") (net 2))
 (segment (start 126.625 61.24553) (end 126.625 62.0068) (width 0.2) (layer "F.Cu") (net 2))
 (segment (start 130.728493 62.645) (end 130.94 62.645) (width 0.2) (layer "F.Cu") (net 2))
 (segment (start 127.2932 62.675) (end 128.5 62.675) (width 0.2) (layer "F.Cu") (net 2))
 (segment (start 129.35 61.35) (end 130.675 62.675) (width 0.2) (layer "F.Cu") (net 2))
 (segment (start 130.675 62.675) (end 130.698493 62.675) (width 0.2) (layer "F.Cu") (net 2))
 (segment (start 130.900699 63.095) (end 130.94 63.095) (width 0.2) (layer "F.Cu") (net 1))
 (segment (start 130.94 63.095) (end 131.35 63.505) (width 0.2) (layer "F.Cu") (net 1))
 (segment (start 126.175 61.43193) (end 126.175 62.1932) (width 0.2) (layer "F.Cu") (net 1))
 (segment (start 127.1068 63.125) (end 128.5 63.125) (width 0.2) (layer "F.Cu") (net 1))
 (segment (start 125.56807 60.825) (end 126.175 61.43193) (width 0.2) (layer "F.Cu") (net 1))
 (segment (start 129.35 63.975) (end 129.35 64.45) (width 0.2) (layer "F.Cu") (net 1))
 (segment (start 130.870699 63.125) (end 130.900699 63.095) (width 0.2) (layer "F.Cu") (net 1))
 (segment (start 124.625 60.825) (end 125.56807 60.825) (width 0.2) (layer "F.Cu") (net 1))
 (segment (start 122.35 63.1) (end 124.625 60.825) (width 0.2) (layer "F.Cu") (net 1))
 (segment (start 126.175 62.1932) (end 127.1068 63.125) (width 0.2) (layer "F.Cu") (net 1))
 (segment (start 130.675 63.125) (end 130.870699 63.125) (width 0.2) (layer "F.Cu") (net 1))
 (segment (start 131.35 63.505) (end 131.789 63.505) (width 0.2) (layer "F.Cu") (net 1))
 (segment (start 128.5 63.125) (end 129.35 63.975) (width 0.2) (layer "F.Cu") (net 1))
 (segment (start 129.35 64.45) (end 130.675 63.125) (width 0.2) (layer "F.Cu") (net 1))
 (segment (start 136.1 53.4) (end 136.1 50.68) (width 0.3) (layer "F.Cu") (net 9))
 (segment (start 144.875 50.427943) (end 145.55181 51.104753) (width 0.3) (layer "F.Cu") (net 9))
 (segment (start 144.875 49.375) (end 145.75 48.5) (width 0.3) (layer "F.Cu") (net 9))
 (segment (start 146.5 48.5) (end 145.75 48.5) (width 0.3) (layer "F.Cu") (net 9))
 (segment (start 137.75 48.5) (end 137.75 49.61) (width 0.3) (layer "F.Cu") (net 9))
 (segment (start 149.2 43.65) (end 148.725 43.65) (width 0.3) (layer "F.Cu") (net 9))
 (segment (start 144.875 50.427943) (end 144.875 49.375) (width 0.3) (layer "F.Cu") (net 9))
 (segment (start 147.5 47.5) (end 146.5 48.5) (width 0.3) (layer "F.Cu") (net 9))
 (segment (start 148.725 43.65) (end 147.5 44.875) (width 0.3) (layer "F.Cu") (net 9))
 (segment (start 137.75 49.61) (end 136.68 50.68) (width 0.3) (layer "F.Cu") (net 9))
 (segment (start 136.68 50.68) (end 136.1 50.68) (width 0.3) (layer "F.Cu") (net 9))
 (segment (start 147.5 44.875) (end 147.5 47.5) (width 0.3) (layer "F.Cu") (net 9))
 (via (at 137.75 48.5) (size 0.9) (drill 0.35) (layers "F.Cu" "B.Cu") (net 9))
 (via (at 145.75 48.5) (size 0.9) (drill 0.35) (layers "F.Cu" "B.Cu") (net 9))
 (segment (start 137.75 48.5) (end 145.75 48.5) (width 0.3) (layer "B.Cu") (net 9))
 (segment (start 148.2 43) (end 146.45 44.75) (width 0.3) (layer "F.Cu") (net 12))
 (segment (start 149.2 43) (end 148.2 43) (width 0.3) (layer "F.Cu") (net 12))
 (segment (start 136.1 44.2) (end 136.1 46.87) (width 0.3) (layer "F.Cu") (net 12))
 (segment (start 137.83 47.5) (end 143.25 47.5) (width 0.3) (layer "F.Cu") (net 12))
 (segment (start 143.25 47.5) (end 144.25 48.5) (width 0.3) (layer "F.Cu") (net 12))
 (segment (start 146 47.7) (end 145.05 47.7) (width 0.3) (layer "F.Cu") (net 12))
 (segment (start 137.2 46.87) (end 137.83 47.5) (width 0.3) (layer "F.Cu") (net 12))
 (segment (start 146.45 47.25) (end 146 47.7) (width 0.3) (layer "F.Cu") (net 12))
 (segment (start 136.1 46.87) (end 137.2 46.87) (width 0.3) (layer "F.Cu") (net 12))
 (segment (start 146.45 44.75) (end 146.45 47.25) (width 0.3) (layer "F.Cu") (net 12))
 (segment (start 145.05 47.7) (end 144.25 48.5) (width 0.3) (layer "F.Cu") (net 12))
 (segment (start 144.25 50.934314) (end 144.977639 51.661953) (width 0.3) (layer "F.Cu") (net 12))
 (segment (start 144.25 48.5) (end 144.25 50.934314) (width 0.3) (layer "F.Cu") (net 12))
 (segment (start 144.375 51.059315) (end 144.986124 51.670439) (width 0.3) (layer "F.Cu") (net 12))
 (segment (start 154.45 43) (end 155 42.45) (width 0.25) (layer "F.Cu") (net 13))
 (segment (start 151 43) (end 154.45 43) (width 0.25) (layer "F.Cu") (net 13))
 (segment (start 150.35 42.35) (end 151 43) (width 0.25) (layer "F.Cu") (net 13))
 (segment (start 149.2 42.35) (end 150.35 42.35) (width 0.25) (layer "F.Cu") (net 13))
 (segment (start 146.5 63) (end 146.5 60.109798) (width 0.25) (layer "F.Cu") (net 10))
 (segment (start 146.5 60.109798) (end 146.674695 59.935103) (width 0.25) (layer "F.Cu") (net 10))
 (segment (start 146.957017 63.457017) (end 146.5 63) (width 0.25) (layer "F.Cu") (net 10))
 (segment (start 146.957017 66.755724) (end 146.51066 67.202081) (width 0.25) (layer "F.Cu") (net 10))
 (segment (start 146.957017 63.457017) (end 146.957017 66.755724) (width 0.25) (layer "F.Cu") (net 10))
 (segment (start 143.8 63.457017) (end 143.8 61.678427) (width 0.25) (layer "F.Cu") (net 11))
 (segment (start 143.8 63.457017) (end 143.8 66.329899) (width 0.25) (layer "F.Cu") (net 11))
 (segment (start 143.8 61.678427) (end 146.10901 59.369417) (width 0.25) (layer "F.Cu") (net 11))
 (segment (start 143.8 66.329899) (end 144.38934 66.919239) (width 0.25) (layer "F.Cu") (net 11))
 (segment (start 158.678427 63.1) (end 163.2 63.1) (width 0.3) (layer "F.Cu") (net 4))
 (segment (start 152.110932 56.532505) (end 158.678427 63.1) (width 0.3) (layer "F.Cu") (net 4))
 (segment (start 163.2 58.1) (end 154.809798 58.1) (width 0.3) (layer "F.Cu") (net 5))
 (segment (start 154.809798 58.1) (end 152.676618 55.96682) (width 0.3) (layer "F.Cu") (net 5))
 (segment (start 152.676618 55.96682) (end 152.676618 55.976618) (width 0.3) (layer "F.Cu") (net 5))
 (segment (start 152.676618 53.93318) (end 162.36682 53.93318) (width 0.3) (layer "F.Cu") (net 6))
 (segment (start 162.36682 53.93318) (end 163.2 53.1) (width 0.3) (layer "F.Cu") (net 6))
 (segment (start 144.420439 52.235419) (end 143.21751 51.03249) (width 0.3) (layer "F.Cu") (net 7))
 (segment (start 142 49.81498) (end 143.21751 51.03249) (width 0.3) (layer "F.Cu") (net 7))
 (segment (start 144.420439 52.236124) (end 144.420439 52.235419) (width 0.3) (layer "F.Cu") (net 7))
 (segment (start 142 49.3) (end 142 49.81498) (width 0.3) (layer "F.Cu") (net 7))
 (via (at 143.21751 51.03249) (size 0.9) (drill 0.35) (layers "F.Cu" "B.Cu") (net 7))
 (segment (start 160.26751 51.03249) (end 163.2 48.1) (width 0.3) (layer "B.Cu") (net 7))
 (segment (start 143.21751 51.03249) (end 160.26751 51.03249) (width 0.3) (layer "B.Cu") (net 7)))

